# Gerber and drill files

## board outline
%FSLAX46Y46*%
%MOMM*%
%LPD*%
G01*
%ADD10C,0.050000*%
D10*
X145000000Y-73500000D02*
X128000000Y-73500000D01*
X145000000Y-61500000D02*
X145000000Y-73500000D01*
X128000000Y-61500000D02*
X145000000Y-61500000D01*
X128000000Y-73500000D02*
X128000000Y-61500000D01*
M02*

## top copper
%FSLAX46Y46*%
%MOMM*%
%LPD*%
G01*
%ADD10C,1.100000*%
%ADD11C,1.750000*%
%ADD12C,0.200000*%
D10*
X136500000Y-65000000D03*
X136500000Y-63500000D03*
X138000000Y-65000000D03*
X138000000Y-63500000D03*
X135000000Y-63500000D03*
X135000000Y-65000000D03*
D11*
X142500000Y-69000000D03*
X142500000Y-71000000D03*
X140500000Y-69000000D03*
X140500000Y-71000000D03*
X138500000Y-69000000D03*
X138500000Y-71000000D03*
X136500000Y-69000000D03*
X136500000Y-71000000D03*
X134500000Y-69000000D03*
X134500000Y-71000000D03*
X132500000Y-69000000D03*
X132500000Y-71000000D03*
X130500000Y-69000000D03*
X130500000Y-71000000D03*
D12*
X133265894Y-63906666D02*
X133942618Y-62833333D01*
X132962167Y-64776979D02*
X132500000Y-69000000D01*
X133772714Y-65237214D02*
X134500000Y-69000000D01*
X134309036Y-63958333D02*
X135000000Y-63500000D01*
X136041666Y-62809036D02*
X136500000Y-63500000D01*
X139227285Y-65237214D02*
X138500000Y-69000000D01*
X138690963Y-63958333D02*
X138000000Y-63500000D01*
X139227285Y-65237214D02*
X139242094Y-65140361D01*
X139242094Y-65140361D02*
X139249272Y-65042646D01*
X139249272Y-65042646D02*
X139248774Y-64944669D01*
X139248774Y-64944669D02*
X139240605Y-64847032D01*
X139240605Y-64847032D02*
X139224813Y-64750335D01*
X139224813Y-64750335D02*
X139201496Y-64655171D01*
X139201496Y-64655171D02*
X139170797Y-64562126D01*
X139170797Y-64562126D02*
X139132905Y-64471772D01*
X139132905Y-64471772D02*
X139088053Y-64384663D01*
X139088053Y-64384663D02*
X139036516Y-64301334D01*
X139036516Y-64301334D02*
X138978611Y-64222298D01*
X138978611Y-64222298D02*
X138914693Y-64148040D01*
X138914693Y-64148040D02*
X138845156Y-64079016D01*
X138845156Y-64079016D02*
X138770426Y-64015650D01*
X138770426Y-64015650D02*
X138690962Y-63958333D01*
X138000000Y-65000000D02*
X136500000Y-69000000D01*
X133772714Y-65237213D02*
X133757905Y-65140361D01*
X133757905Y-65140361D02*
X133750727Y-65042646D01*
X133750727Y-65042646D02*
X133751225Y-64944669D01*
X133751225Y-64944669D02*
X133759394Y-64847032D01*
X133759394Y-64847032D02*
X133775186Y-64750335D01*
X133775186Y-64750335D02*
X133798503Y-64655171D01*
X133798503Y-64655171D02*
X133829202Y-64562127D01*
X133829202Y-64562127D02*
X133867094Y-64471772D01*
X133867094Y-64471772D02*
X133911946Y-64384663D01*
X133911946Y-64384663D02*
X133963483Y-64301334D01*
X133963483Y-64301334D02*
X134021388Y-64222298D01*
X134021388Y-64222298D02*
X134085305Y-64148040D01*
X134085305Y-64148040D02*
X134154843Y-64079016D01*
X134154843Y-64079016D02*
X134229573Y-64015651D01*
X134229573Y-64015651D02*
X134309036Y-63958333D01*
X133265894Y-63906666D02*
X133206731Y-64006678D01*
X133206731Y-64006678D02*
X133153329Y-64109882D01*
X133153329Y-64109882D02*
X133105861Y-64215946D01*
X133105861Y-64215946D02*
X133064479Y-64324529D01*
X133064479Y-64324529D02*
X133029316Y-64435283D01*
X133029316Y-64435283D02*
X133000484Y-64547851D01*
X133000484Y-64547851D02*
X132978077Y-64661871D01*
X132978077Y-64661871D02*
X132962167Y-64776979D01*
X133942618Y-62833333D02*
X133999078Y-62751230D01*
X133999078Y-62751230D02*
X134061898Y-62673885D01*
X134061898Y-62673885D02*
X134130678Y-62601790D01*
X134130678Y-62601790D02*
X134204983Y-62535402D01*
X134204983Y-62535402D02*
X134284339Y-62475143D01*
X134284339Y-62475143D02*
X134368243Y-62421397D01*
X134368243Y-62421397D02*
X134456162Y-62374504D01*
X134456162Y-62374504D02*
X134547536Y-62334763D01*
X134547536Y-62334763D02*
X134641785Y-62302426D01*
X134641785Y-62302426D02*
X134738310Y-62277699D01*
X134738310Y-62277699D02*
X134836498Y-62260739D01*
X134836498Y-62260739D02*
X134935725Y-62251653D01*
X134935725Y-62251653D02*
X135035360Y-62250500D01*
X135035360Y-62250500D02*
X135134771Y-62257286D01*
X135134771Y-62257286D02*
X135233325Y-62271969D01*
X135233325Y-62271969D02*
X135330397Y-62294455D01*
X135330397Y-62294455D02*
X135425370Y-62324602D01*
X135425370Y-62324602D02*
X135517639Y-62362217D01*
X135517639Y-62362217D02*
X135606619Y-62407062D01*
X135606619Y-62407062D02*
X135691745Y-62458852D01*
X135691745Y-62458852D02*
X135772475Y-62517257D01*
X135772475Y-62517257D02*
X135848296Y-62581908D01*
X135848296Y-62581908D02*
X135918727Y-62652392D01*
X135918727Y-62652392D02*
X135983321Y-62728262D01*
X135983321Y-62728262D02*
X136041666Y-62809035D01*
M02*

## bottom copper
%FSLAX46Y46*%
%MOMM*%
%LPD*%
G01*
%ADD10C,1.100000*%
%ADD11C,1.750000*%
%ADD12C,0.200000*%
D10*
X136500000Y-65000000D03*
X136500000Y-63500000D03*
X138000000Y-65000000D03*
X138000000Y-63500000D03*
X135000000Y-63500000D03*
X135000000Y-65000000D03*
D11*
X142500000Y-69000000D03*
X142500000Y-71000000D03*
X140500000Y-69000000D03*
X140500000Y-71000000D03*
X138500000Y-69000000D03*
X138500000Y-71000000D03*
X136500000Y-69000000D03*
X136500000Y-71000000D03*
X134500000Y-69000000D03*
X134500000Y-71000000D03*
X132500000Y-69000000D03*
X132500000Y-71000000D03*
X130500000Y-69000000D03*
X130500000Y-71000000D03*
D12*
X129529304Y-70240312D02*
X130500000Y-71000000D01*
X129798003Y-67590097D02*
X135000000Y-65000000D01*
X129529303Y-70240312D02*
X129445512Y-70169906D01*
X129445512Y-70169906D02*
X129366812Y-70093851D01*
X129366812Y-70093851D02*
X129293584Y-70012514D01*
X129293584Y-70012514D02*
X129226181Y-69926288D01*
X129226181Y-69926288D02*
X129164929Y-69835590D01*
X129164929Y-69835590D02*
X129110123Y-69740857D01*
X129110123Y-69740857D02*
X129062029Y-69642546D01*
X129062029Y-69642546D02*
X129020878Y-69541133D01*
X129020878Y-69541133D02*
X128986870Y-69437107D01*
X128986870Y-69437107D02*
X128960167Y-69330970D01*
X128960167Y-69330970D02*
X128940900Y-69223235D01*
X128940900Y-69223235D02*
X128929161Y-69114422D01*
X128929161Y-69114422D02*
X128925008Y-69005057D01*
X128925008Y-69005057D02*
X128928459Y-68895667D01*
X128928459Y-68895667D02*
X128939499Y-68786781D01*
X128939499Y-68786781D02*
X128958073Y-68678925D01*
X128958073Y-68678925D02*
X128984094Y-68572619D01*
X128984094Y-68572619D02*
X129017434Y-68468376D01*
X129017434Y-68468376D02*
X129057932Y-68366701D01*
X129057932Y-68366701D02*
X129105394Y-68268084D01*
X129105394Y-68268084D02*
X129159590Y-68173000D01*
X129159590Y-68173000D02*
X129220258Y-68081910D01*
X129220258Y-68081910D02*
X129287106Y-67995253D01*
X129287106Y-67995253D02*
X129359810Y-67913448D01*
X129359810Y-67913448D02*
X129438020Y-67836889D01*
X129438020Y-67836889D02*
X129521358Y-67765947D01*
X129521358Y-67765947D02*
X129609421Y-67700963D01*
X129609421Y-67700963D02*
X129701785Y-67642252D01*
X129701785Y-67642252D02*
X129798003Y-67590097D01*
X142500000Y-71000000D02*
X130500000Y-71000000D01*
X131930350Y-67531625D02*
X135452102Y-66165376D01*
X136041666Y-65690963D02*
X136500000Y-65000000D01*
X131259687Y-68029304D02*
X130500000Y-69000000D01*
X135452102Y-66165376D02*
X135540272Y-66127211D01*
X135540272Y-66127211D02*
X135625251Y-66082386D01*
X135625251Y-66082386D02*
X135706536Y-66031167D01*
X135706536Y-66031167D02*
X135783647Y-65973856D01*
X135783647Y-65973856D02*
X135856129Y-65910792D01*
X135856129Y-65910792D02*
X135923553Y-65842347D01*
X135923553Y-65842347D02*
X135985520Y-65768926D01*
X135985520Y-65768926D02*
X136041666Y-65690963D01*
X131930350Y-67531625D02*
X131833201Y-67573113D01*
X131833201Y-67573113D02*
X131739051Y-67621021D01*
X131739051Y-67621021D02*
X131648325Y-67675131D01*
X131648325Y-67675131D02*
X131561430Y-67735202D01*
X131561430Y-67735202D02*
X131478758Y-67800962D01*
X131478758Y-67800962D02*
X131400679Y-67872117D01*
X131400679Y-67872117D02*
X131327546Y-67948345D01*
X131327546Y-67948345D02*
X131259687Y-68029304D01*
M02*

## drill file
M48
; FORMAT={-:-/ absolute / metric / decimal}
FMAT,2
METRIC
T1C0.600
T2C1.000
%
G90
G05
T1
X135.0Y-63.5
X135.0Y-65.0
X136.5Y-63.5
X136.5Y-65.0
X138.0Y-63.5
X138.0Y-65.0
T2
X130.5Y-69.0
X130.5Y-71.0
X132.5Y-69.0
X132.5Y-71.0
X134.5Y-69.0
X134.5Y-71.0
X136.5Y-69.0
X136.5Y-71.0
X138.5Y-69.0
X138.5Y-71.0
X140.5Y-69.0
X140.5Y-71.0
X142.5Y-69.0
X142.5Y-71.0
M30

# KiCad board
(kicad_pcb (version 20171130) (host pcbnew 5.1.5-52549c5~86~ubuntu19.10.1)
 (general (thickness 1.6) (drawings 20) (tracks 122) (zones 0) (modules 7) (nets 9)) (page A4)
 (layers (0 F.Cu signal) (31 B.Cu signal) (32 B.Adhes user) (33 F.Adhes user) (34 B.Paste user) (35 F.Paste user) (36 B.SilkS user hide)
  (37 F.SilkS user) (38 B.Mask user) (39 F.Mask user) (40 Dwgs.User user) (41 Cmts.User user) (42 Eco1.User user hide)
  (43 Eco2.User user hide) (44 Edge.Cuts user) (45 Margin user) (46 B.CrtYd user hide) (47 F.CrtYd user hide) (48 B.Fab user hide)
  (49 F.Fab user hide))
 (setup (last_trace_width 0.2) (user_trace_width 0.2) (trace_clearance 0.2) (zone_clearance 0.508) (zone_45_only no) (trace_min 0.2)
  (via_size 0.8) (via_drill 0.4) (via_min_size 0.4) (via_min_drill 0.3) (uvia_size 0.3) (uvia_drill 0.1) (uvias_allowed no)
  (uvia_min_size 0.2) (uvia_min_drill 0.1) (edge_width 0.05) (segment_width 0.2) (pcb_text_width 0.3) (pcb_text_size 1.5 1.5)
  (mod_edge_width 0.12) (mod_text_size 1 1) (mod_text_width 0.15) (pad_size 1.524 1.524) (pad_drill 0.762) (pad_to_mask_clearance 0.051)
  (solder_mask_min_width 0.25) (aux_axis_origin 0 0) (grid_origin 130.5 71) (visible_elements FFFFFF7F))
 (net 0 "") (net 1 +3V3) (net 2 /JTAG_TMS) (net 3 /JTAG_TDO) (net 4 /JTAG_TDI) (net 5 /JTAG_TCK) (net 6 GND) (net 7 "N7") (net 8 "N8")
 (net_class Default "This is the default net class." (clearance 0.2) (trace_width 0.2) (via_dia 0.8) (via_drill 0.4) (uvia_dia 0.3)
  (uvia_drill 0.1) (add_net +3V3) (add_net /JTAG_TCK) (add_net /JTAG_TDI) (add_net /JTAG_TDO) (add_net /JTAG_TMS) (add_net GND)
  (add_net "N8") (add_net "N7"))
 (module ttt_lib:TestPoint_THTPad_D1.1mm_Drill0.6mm (layer B.Cu) (at 136.5 65)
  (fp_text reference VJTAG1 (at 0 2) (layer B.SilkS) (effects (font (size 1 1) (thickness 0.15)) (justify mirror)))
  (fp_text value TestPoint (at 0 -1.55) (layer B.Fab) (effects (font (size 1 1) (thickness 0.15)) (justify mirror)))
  (pad 1 thru_hole circle (at 0 0) (size 1.1 1.1) (drill 0.6) (layers *.Cu *.Mask) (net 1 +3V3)))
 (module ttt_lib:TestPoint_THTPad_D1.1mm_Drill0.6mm (layer B.Cu) (at 136.5 63.5)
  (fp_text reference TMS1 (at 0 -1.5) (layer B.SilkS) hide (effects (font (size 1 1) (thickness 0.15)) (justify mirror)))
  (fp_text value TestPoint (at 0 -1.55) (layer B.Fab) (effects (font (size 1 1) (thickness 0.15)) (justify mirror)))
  (pad 1 thru_hole circle (at 0 0) (size 1.1 1.1) (drill 0.6) (layers *.Cu *.Mask) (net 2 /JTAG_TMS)))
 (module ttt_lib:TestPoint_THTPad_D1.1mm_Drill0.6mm (layer B.Cu) (at 138 65)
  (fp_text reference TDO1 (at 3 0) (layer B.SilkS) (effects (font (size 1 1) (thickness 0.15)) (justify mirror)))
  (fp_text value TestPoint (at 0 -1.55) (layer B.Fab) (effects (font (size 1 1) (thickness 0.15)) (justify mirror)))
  (pad 1 thru_hole circle (at 0 0) (size 1.1 1.1) (drill 0.6) (layers *.Cu *.Mask) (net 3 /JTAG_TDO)))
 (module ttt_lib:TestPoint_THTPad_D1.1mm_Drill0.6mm (layer B.Cu) (at 138 63.5)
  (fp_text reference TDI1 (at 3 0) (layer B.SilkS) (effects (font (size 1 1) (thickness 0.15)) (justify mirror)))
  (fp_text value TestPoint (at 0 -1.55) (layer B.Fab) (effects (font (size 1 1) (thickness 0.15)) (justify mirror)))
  (pad 1 thru_hole circle (at 0 0) (size 1.1 1.1) (drill 0.6) (layers *.Cu *.Mask) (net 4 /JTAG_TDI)))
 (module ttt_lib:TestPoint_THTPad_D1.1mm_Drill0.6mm (layer B.Cu) (at 135 63.5)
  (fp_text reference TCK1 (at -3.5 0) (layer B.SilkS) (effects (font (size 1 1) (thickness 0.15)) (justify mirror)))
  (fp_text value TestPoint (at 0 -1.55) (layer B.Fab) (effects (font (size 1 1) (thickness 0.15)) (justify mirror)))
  (pad 1 thru_hole circle (at 0 0) (size 1.1 1.1) (drill 0.6) (layers *.Cu *.Mask) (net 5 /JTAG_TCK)))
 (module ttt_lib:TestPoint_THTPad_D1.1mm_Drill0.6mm (layer B.Cu) (at 135 65)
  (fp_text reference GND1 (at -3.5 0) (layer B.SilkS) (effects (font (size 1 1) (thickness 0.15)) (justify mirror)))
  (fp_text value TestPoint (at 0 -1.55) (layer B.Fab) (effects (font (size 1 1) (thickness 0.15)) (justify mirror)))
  (pad 1 thru_hole circle (at 0 0) (size 1.1 1.1) (drill 0.6) (layers *.Cu *.Mask) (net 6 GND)))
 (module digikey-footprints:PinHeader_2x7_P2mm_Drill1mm (layer F.Cu) (at 130.5 71 180)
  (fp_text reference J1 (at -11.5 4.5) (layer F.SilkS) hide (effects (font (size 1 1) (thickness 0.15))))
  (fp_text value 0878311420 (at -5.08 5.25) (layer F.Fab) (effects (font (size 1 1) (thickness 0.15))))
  (pad 14 thru_hole circle (at -12 2 180) (size 1.75 1.75) (drill 1) (layers *.Cu *.Mask) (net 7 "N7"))
  (pad 13 thru_hole circle (at -12 0 180) (size 1.75 1.75) (drill 1) (layers *.Cu *.Mask) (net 6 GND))
  (pad 12 thru_hole circle (at -10 2 180) (size 1.75 1.75) (drill 1) (layers *.Cu *.Mask) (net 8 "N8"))
  (pad 11 thru_hole circle (at -10 0 180) (size 1.75 1.75) (drill 1) (layers *.Cu *.Mask) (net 6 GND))
  (pad 10 thru_hole circle (at -8 2 180) (size 1.75 1.75) (drill 1) (layers *.Cu *.Mask) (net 4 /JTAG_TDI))
  (pad 9 thru_hole circle (at -8 0 180) (size 1.75 1.75) (drill 1) (layers *.Cu *.Mask) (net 6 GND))
  (pad 8 thru_hole circle (at -6 2 180) (size 1.75 1.75) (drill 1) (layers *.Cu *.Mask) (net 3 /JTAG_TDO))
  (pad 7 thru_hole circle (at -6 0 180) (size 1.75 1.75) (drill 1) (layers *.Cu *.Mask) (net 6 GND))
  (pad 6 thru_hole circle (at -4 2 180) (size 1.75 1.75) (drill 1) (layers *.Cu *.Mask) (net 5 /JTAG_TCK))
  (pad 5 thru_hole circle (at -4 0 180) (size 1.75 1.75) (drill 1) (layers *.Cu *.Mask) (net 6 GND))
  (pad 4 thru_hole circle (at -2 2 180) (size 1.75 1.75) (drill 1) (layers *.Cu *.Mask) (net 2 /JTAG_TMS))
  (pad 3 thru_hole circle (at -2 0 180) (size 1.75 1.75) (drill 1) (layers *.Cu *.Mask) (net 6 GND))
  (pad 2 thru_hole circle (at 0 2 180) (size 1.75 1.75) (drill 1) (layers *.Cu *.Mask) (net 1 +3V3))
  (pad 1 thru_hole circle (at 0 0 180) (size 1.75 1.75) (drill 1) (layers *.Cu *.Mask) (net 6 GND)))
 (gr_line (start 145 73.5) (end 128 73.5) (layer Edge.Cuts) (width 0.05))
 (gr_line (start 145 61.5) (end 145 73.5) (layer Edge.Cuts) (width 0.05))
 (gr_line (start 128 61.5) (end 145 61.5) (layer Edge.Cuts) (width 0.05))
 (gr_line (start 128 73.5) (end 128 61.5) (layer Edge.Cuts) (width 0.05))
 (segment (start 129.529304 70.240312) (end 130.5 71) (width 0.2) (layer B.Cu) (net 6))
 (segment (start 129.798003 67.590097) (end 135 65) (width 0.2) (layer B.Cu) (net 6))
 (segment (start 129.529303 70.240312) (end 129.445512 70.169906) (width 0.2) (layer B.Cu) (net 6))
 (segment (start 129.445512 70.169906) (end 129.366812 70.093851) (width 0.2) (layer B.Cu) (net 6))
 (segment (start 129.366812 70.093851) (end 129.293584 70.012514) (width 0.2) (layer B.Cu) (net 6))
 (segment (start 129.293584 70.012514) (end 129.226181 69.926288) (width 0.2) (layer B.Cu) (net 6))
 (segment (start 129.226181 69.926288) (end 129.164929 69.83559) (width 0.2) (layer B.Cu) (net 6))
 (segment (start 129.164929 69.83559) (end 129.110123 69.740857) (width 0.2) (layer B.Cu) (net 6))
 (segment (start 129.110123 69.740857) (end 129.062029 69.642546) (width 0.2) (layer B.Cu) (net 6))
 (segment (start 129.062029 69.642546) (end 129.020878 69.541133) (width 0.2) (layer B.Cu) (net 6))
 (segment (start 129.020878 69.541133) (end 128.98687 69.437107) (width 0.2) (layer B.Cu) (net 6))
 (segment (start 128.98687 69.437107) (end 128.960167 69.33097) (width 0.2) (layer B.Cu) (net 6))
 (segment (start 128.960167 69.33097) (end 128.9409 69.223235) (width 0.2) (layer B.Cu) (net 6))
 (segment (start 128.9409 69.223235) (end 128.929161 69.114422) (width 0.2) (layer B.Cu) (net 6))
 (segment (start 128.929161 69.114422) (end 128.925008 69.005057) (width 0.2) (layer B.Cu) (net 6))
 (segment (start 128.925008 69.005057) (end 128.928459 68.895667) (width 0.2) (layer B.Cu) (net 6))
 (segment (start 128.928459 68.895667) (end 128.939499 68.786781) (width 0.2) (layer B.Cu) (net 6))
 (segment (start 128.939499 68.786781) (end 128.958073 68.678925) (width 0.2) (layer B.Cu) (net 6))
 (segment (start 128.958073 68.678925) (end 128.984094 68.572619) (width 0.2) (layer B.Cu) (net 6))
 (segment (start 128.984094 68.572619) (end 129.017434 68.468376) (width 0.2) (layer B.Cu) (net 6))
 (segment (start 129.017434 68.468376) (end 129.057932 68.366701) (width 0.2) (layer B.Cu) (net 6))
 (segment (start 129.057932 68.366701) (end 129.105394 68.268084) (width 0.2) (layer B.Cu) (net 6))
 (segment (start 129.105394 68.268084) (end 129.15959 68.173) (width 0.2) (layer B.Cu) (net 6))
 (segment (start 129.15959 68.173) (end 129.220258 68.08191) (width 0.2) (layer B.Cu) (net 6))
 (segment (start 129.220258 68.08191) (end 129.287106 67.995253) (width 0.2) (layer B.Cu) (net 6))
 (segment (start 129.287106 67.995253) (end 129.35981 67.913448) (width 0.2) (layer B.Cu) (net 6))
 (segment (start 129.35981 67.913448) (end 129.43802 67.836889) (width 0.2) (layer B.Cu) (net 6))
 (segment (start 129.43802 67.836889) (end 129.521358 67.765947) (width 0.2) (layer B.Cu) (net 6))
 (segment (start 129.521358 67.765947) (end 129.609421 67.700963) (width 0.2) (layer B.Cu) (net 6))
 (segment (start 129.609421 67.700963) (end 129.701785 67.642252) (width 0.2) (layer B.Cu) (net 6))
 (segment (start 129.701785 67.642252) (end 129.798003 67.590097) (width 0.2) (layer B.Cu) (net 6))
 (segment (start 142.5 71) (end 130.5 71) (width 0.2) (layer B.Cu) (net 6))
 (segment (start 131.93035 67.531625) (end 135.452102 66.165376) (width 0.2) (layer B.Cu) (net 1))
 (segment (start 136.041666 65.690963) (end 136.5 65) (width 0.2) (layer B.Cu) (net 1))
 (segment (start 131.259687 68.029304) (end 130.5 69) (width 0.2) (layer B.Cu) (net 1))
 (segment (start 133.265894 63.906666) (end 133.942618 62.833333) (width 0.2) (layer F.Cu) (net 2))
 (segment (start 132.962167 64.776979) (end 132.5 69) (width 0.2) (layer F.Cu) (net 2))
 (segment (start 133.772714 65.237214) (end 134.5 69) (width 0.2) (layer F.Cu) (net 5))
 (segment (start 134.309036 63.958333) (end 135 63.5) (width 0.2) (layer F.Cu) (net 5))
 (segment (start 136.041666 62.809036) (end 136.5 63.5) (width 0.2) (layer F.Cu) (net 2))
 (segment (start 139.227285 65.237214) (end 138.5 69) (width 0.2) (layer F.Cu) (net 4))
 (segment (start 138.690963 63.958333) (end 138 63.5) (width 0.2) (layer F.Cu) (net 4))
 (segment (start 139.227285 65.237214) (end 139.242094 65.140361) (width 0.2) (layer F.Cu) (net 4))
 (segment (start 139.242094 65.140361) (end 139.249272 65.042646) (width 0.2) (layer F.Cu) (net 4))
 (segment (start 139.249272 65.042646) (end 139.248774 64.944669) (width 0.2) (layer F.Cu) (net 4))
 (segment (start 139.248774 64.944669) (end 139.240605 64.847032) (width 0.2) (layer F.Cu) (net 4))
 (segment (start 139.240605 64.847032) (end 139.224813 64.750335) (width 0.2) (layer F.Cu) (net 4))
 (segment (start 139.224813 64.750335) (end 139.201496 64.655171) (width 0.2) (layer F.Cu) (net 4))
 (segment (start 139.201496 64.655171) (end 139.170797 64.562126) (width 0.2) (layer F.Cu) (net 4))
 (segment (start 139.170797 64.562126) (end 139.132905 64.471772) (width 0.2) (layer F.Cu) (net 4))
 (segment (start 139.132905 64.471772) (end 139.088053 64.384663) (width 0.2) (layer F.Cu) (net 4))
 (segment (start 139.088053 64.384663) (end 139.036516 64.301334) (width 0.2) (layer F.Cu) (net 4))
 (segment (start 139.036516 64.301334) (end 138.978611 64.222298) (width 0.2) (layer F.Cu) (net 4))
 (segment (start 138.978611 64.222298) (end 138.914693 64.14804) (width 0.2) (layer F.Cu) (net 4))
 (segment (start 138.914693 64.14804) (end 138.845156 64.079016) (width 0.2) (layer F.Cu) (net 4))
 (segment (start 138.845156 64.079016) (end 138.770426 64.01565) (width 0.2) (layer F.Cu) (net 4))
 (segment (start 138.770426 64.01565) (end 138.690962 63.958333) (width 0.2) (layer F.Cu) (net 4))
 (segment (start 138 65) (end 136.5 69) (width 0.2) (layer F.Cu) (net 3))
 (segment (start 133.772714 65.237213) (end 133.757905 65.140361) (width 0.2) (layer F.Cu) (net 5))
 (segment (start 133.757905 65.140361) (end 133.750727 65.042646) (width 0.2) (layer F.Cu) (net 5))
 (segment (start 133.750727 65.042646) (end 133.751225 64.944669) (width 0.2) (layer F.Cu) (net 5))
 (segment (start 133.751225 64.944669) (end 133.759394 64.847032) (width 0.2) (layer F.Cu) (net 5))
 (segment (start 133.759394 64.847032) (end 133.775186 64.750335) (width 0.2) (layer F.Cu) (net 5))
 (segment (start 133.775186 64.750335) (end 133.798503 64.655171) (width 0.2) (layer F.Cu) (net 5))
 (segment (start 133.798503 64.655171) (end 133.829202 64.562127) (width 0.2) (layer F.Cu) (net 5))
 (segment (start 133.829202 64.562127) (end 133.867094 64.471772) (width 0.2) (layer F.Cu) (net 5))
 (segment (start 133.867094 64.471772) (end 133.911946 64.384663) (width 0.2) (layer F.Cu) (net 5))
 (segment (start 133.911946 64.384663) (end 133.963483 64.301334) (width 0.2) (layer F.Cu) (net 5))
 (segment (start 133.963483 64.301334) (end 134.021388 64.222298) (width 0.2) (layer F.Cu) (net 5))
 (segment (start 134.021388 64.222298) (end 134.085305 64.14804) (width 0.2) (layer F.Cu) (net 5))
 (segment (start 134.085305 64.14804) (end 134.154843 64.079016) (width 0.2) (layer F.Cu) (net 5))
 (segment (start 134.154843 64.079016) (end 134.229573 64.015651) (width 0.2) (layer F.Cu) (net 5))
 (segment (start 134.229573 64.015651) (end 134.309036 63.958333) (width 0.2) (layer F.Cu) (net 5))
 (segment (start 133.265894 63.906666) (end 133.206731 64.006678) (width 0.2) (layer F.Cu) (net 2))
 (segment (start 133.206731 64.006678) (end 133.153329 64.109882) (width 0.2) (layer F.Cu) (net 2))
 (segment (start 133.153329 64.109882) (end 133.105861 64.215946) (width 0.2) (layer F.Cu) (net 2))
 (segment (start 133.105861 64.215946) (end 133.064479 64.324529) (width 0.2) (layer F.Cu) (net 2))
 (segment (start 133.064479 64.324529) (end 133.029316 64.435283) (width 0.2) (layer F.Cu) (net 2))
 (segment (start 133.029316 64.435283) (end 133.000484 64.547851) (width 0.2) (layer F.Cu) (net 2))
 (segment (start 133.000484 64.547851) (end 132.978077 64.661871) (width 0.2) (layer F.Cu) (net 2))
 (segment (start 132.978077 64.661871) (end 132.962167 64.776979) (width 0.2) (layer F.Cu) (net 2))
 (segment (start 133.942618 62.833333) (end 133.999078 62.75123) (width 0.2) (layer F.Cu) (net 2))
 (segment (start 133.999078 62.75123) (end 134.061898 62.673885) (width 0.2) (layer F.Cu) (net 2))
 (segment (start 134.061898 62.673885) (end 134.130678 62.60179) (width 0.2) (layer F.Cu) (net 2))
 (segment (start 134.130678 62.60179) (end 134.204983 62.535402) (width 0.2) (layer F.Cu) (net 2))
 (segment (start 134.204983 62.535402) (end 134.284339 62.475143) (width 0.2) (layer F.Cu) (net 2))
 (segment (start 134.284339 62.475143) (end 134.368243 62.421397) (width 0.2) (layer F.Cu) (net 2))
 (segment (start 134.368243 62.421397) (end 134.456162 62.374504) (width 0.2) (layer F.Cu) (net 2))
 (segment (start 134.456162 62.374504) (end 134.547536 62.334763) (width 0.2) (layer F.Cu) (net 2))
 (segment (start 134.547536 62.334763) (end 134.641785 62.302426) (width 0.2) (layer F.Cu) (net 2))
 (segment (start 134.641785 62.302426) (end 134.73831 62.277699) (width 0.2) (layer F.Cu) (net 2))
 (segment (start 134.73831 62.277699) (end 134.836498 62.260739) (width 0.2) (layer F.Cu) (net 2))
 (segment (start 134.836498 62.260739) (end 134.935725 62.251653) (width 0.2) (layer F.Cu) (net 2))
 (segment (start 134.935725 62.251653) (end 135.03536 62.2505) (width 0.2) (layer F.Cu) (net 2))
 (segment (start 135.03536 62.2505) (end 135.134771 62.257286) (width 0.2) (layer F.Cu) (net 2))
 (segment (start 135.134771 62.257286) (end 135.233325 62.271969) (width 0.2) (layer F.Cu) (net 2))
 (segment (start 135.233325 62.271969) (end 135.330397 62.294455) (width 0.2) (layer F.Cu) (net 2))
 (segment (start 135.330397 62.294455) (end 135.42537 62.324602) (width 0.2) (layer F.Cu) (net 2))
 (segment (start 135.42537 62.324602) (end 135.517639 62.362217) (width 0.2) (layer F.Cu) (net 2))
 (segment (start 135.517639 62.362217) (end 135.606619 62.407062) (width 0.2) (layer F.Cu) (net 2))
 (segment (start 135.606619 62.407062) (end 135.691745 62.458852) (width 0.2) (layer F.Cu) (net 2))
 (segment (start 135.691745 62.458852) (end 135.772475 62.517257) (width 0.2) (layer F.Cu) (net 2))
 (segment (start 135.772475 62.517257) (end 135.848296 62.581908) (width 0.2) (layer F.Cu) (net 2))
 (segment (start 135.848296 62.581908) (end 135.918727 62.652392) (width 0.2) (layer F.Cu) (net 2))
 (segment (start 135.918727 62.652392) (end 135.983321 62.728262) (width 0.2) (layer F.Cu) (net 2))
 (segment (start 135.983321 62.728262) (end 136.041666 62.809035) (width 0.2) (layer F.Cu) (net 2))
 (segment (start 135.452102 66.165376) (end 135.540272 66.127211) (width 0.2) (layer B.Cu) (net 1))
 (segment (start 135.540272 66.127211) (end 135.625251 66.082386) (width 0.2) (layer B.Cu) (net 1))
 (segment (start 135.625251 66.082386) (end 135.706536 66.031167) (width 0.2) (layer B.Cu) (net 1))
 (segment (start 135.706536 66.031167) (end 135.783647 65.973856) (width 0.2) (layer B.Cu) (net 1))
 (segment (start 135.783647 65.973856) (end 135.856129 65.910792) (width 0.2) (layer B.Cu) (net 1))
 (segment (start 135.856129 65.910792) (end 135.923553 65.842347) (width 0.2) (layer B.Cu) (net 1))
 (segment (start 135.923553 65.842347) (end 135.98552 65.768926) (width 0.2) (layer B.Cu) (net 1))
 (segment (start 135.98552 65.768926) (end 136.041666 65.690963) (width 0.2) (layer B.Cu) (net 1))
 (segment (start 131.93035 67.531625) (end 131.833201 67.573113) (width 0.2) (layer B.Cu) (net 1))
 (segment (start 131.833201 67.573113) (end 131.739051 67.621021) (width 0.2) (layer B.Cu) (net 1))
 (segment (start 131.739051 67.621021) (end 131.648325 67.675131) (width 0.2) (layer B.Cu) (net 1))
 (segment (start 131.648325 67.675131) (end 131.56143 67.735202) (width 0.2) (layer B.Cu) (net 1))
 (segment (start 131.56143 67.735202) (end 131.478758 67.800962) (width 0.2) (layer B.Cu) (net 1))
 (segment (start 131.478758 67.800962) (end 131.400679 67.872117) (width 0.2) (layer B.Cu) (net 1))
 (segment (start 131.400679 67.872117) (end 131.327546 67.948345) (width 0.2) (layer B.Cu) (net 1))
 (segment (start 131.327546 67.948345) (end 131.259687 68.029304) (width 0.2) (layer B.Cu) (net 1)))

